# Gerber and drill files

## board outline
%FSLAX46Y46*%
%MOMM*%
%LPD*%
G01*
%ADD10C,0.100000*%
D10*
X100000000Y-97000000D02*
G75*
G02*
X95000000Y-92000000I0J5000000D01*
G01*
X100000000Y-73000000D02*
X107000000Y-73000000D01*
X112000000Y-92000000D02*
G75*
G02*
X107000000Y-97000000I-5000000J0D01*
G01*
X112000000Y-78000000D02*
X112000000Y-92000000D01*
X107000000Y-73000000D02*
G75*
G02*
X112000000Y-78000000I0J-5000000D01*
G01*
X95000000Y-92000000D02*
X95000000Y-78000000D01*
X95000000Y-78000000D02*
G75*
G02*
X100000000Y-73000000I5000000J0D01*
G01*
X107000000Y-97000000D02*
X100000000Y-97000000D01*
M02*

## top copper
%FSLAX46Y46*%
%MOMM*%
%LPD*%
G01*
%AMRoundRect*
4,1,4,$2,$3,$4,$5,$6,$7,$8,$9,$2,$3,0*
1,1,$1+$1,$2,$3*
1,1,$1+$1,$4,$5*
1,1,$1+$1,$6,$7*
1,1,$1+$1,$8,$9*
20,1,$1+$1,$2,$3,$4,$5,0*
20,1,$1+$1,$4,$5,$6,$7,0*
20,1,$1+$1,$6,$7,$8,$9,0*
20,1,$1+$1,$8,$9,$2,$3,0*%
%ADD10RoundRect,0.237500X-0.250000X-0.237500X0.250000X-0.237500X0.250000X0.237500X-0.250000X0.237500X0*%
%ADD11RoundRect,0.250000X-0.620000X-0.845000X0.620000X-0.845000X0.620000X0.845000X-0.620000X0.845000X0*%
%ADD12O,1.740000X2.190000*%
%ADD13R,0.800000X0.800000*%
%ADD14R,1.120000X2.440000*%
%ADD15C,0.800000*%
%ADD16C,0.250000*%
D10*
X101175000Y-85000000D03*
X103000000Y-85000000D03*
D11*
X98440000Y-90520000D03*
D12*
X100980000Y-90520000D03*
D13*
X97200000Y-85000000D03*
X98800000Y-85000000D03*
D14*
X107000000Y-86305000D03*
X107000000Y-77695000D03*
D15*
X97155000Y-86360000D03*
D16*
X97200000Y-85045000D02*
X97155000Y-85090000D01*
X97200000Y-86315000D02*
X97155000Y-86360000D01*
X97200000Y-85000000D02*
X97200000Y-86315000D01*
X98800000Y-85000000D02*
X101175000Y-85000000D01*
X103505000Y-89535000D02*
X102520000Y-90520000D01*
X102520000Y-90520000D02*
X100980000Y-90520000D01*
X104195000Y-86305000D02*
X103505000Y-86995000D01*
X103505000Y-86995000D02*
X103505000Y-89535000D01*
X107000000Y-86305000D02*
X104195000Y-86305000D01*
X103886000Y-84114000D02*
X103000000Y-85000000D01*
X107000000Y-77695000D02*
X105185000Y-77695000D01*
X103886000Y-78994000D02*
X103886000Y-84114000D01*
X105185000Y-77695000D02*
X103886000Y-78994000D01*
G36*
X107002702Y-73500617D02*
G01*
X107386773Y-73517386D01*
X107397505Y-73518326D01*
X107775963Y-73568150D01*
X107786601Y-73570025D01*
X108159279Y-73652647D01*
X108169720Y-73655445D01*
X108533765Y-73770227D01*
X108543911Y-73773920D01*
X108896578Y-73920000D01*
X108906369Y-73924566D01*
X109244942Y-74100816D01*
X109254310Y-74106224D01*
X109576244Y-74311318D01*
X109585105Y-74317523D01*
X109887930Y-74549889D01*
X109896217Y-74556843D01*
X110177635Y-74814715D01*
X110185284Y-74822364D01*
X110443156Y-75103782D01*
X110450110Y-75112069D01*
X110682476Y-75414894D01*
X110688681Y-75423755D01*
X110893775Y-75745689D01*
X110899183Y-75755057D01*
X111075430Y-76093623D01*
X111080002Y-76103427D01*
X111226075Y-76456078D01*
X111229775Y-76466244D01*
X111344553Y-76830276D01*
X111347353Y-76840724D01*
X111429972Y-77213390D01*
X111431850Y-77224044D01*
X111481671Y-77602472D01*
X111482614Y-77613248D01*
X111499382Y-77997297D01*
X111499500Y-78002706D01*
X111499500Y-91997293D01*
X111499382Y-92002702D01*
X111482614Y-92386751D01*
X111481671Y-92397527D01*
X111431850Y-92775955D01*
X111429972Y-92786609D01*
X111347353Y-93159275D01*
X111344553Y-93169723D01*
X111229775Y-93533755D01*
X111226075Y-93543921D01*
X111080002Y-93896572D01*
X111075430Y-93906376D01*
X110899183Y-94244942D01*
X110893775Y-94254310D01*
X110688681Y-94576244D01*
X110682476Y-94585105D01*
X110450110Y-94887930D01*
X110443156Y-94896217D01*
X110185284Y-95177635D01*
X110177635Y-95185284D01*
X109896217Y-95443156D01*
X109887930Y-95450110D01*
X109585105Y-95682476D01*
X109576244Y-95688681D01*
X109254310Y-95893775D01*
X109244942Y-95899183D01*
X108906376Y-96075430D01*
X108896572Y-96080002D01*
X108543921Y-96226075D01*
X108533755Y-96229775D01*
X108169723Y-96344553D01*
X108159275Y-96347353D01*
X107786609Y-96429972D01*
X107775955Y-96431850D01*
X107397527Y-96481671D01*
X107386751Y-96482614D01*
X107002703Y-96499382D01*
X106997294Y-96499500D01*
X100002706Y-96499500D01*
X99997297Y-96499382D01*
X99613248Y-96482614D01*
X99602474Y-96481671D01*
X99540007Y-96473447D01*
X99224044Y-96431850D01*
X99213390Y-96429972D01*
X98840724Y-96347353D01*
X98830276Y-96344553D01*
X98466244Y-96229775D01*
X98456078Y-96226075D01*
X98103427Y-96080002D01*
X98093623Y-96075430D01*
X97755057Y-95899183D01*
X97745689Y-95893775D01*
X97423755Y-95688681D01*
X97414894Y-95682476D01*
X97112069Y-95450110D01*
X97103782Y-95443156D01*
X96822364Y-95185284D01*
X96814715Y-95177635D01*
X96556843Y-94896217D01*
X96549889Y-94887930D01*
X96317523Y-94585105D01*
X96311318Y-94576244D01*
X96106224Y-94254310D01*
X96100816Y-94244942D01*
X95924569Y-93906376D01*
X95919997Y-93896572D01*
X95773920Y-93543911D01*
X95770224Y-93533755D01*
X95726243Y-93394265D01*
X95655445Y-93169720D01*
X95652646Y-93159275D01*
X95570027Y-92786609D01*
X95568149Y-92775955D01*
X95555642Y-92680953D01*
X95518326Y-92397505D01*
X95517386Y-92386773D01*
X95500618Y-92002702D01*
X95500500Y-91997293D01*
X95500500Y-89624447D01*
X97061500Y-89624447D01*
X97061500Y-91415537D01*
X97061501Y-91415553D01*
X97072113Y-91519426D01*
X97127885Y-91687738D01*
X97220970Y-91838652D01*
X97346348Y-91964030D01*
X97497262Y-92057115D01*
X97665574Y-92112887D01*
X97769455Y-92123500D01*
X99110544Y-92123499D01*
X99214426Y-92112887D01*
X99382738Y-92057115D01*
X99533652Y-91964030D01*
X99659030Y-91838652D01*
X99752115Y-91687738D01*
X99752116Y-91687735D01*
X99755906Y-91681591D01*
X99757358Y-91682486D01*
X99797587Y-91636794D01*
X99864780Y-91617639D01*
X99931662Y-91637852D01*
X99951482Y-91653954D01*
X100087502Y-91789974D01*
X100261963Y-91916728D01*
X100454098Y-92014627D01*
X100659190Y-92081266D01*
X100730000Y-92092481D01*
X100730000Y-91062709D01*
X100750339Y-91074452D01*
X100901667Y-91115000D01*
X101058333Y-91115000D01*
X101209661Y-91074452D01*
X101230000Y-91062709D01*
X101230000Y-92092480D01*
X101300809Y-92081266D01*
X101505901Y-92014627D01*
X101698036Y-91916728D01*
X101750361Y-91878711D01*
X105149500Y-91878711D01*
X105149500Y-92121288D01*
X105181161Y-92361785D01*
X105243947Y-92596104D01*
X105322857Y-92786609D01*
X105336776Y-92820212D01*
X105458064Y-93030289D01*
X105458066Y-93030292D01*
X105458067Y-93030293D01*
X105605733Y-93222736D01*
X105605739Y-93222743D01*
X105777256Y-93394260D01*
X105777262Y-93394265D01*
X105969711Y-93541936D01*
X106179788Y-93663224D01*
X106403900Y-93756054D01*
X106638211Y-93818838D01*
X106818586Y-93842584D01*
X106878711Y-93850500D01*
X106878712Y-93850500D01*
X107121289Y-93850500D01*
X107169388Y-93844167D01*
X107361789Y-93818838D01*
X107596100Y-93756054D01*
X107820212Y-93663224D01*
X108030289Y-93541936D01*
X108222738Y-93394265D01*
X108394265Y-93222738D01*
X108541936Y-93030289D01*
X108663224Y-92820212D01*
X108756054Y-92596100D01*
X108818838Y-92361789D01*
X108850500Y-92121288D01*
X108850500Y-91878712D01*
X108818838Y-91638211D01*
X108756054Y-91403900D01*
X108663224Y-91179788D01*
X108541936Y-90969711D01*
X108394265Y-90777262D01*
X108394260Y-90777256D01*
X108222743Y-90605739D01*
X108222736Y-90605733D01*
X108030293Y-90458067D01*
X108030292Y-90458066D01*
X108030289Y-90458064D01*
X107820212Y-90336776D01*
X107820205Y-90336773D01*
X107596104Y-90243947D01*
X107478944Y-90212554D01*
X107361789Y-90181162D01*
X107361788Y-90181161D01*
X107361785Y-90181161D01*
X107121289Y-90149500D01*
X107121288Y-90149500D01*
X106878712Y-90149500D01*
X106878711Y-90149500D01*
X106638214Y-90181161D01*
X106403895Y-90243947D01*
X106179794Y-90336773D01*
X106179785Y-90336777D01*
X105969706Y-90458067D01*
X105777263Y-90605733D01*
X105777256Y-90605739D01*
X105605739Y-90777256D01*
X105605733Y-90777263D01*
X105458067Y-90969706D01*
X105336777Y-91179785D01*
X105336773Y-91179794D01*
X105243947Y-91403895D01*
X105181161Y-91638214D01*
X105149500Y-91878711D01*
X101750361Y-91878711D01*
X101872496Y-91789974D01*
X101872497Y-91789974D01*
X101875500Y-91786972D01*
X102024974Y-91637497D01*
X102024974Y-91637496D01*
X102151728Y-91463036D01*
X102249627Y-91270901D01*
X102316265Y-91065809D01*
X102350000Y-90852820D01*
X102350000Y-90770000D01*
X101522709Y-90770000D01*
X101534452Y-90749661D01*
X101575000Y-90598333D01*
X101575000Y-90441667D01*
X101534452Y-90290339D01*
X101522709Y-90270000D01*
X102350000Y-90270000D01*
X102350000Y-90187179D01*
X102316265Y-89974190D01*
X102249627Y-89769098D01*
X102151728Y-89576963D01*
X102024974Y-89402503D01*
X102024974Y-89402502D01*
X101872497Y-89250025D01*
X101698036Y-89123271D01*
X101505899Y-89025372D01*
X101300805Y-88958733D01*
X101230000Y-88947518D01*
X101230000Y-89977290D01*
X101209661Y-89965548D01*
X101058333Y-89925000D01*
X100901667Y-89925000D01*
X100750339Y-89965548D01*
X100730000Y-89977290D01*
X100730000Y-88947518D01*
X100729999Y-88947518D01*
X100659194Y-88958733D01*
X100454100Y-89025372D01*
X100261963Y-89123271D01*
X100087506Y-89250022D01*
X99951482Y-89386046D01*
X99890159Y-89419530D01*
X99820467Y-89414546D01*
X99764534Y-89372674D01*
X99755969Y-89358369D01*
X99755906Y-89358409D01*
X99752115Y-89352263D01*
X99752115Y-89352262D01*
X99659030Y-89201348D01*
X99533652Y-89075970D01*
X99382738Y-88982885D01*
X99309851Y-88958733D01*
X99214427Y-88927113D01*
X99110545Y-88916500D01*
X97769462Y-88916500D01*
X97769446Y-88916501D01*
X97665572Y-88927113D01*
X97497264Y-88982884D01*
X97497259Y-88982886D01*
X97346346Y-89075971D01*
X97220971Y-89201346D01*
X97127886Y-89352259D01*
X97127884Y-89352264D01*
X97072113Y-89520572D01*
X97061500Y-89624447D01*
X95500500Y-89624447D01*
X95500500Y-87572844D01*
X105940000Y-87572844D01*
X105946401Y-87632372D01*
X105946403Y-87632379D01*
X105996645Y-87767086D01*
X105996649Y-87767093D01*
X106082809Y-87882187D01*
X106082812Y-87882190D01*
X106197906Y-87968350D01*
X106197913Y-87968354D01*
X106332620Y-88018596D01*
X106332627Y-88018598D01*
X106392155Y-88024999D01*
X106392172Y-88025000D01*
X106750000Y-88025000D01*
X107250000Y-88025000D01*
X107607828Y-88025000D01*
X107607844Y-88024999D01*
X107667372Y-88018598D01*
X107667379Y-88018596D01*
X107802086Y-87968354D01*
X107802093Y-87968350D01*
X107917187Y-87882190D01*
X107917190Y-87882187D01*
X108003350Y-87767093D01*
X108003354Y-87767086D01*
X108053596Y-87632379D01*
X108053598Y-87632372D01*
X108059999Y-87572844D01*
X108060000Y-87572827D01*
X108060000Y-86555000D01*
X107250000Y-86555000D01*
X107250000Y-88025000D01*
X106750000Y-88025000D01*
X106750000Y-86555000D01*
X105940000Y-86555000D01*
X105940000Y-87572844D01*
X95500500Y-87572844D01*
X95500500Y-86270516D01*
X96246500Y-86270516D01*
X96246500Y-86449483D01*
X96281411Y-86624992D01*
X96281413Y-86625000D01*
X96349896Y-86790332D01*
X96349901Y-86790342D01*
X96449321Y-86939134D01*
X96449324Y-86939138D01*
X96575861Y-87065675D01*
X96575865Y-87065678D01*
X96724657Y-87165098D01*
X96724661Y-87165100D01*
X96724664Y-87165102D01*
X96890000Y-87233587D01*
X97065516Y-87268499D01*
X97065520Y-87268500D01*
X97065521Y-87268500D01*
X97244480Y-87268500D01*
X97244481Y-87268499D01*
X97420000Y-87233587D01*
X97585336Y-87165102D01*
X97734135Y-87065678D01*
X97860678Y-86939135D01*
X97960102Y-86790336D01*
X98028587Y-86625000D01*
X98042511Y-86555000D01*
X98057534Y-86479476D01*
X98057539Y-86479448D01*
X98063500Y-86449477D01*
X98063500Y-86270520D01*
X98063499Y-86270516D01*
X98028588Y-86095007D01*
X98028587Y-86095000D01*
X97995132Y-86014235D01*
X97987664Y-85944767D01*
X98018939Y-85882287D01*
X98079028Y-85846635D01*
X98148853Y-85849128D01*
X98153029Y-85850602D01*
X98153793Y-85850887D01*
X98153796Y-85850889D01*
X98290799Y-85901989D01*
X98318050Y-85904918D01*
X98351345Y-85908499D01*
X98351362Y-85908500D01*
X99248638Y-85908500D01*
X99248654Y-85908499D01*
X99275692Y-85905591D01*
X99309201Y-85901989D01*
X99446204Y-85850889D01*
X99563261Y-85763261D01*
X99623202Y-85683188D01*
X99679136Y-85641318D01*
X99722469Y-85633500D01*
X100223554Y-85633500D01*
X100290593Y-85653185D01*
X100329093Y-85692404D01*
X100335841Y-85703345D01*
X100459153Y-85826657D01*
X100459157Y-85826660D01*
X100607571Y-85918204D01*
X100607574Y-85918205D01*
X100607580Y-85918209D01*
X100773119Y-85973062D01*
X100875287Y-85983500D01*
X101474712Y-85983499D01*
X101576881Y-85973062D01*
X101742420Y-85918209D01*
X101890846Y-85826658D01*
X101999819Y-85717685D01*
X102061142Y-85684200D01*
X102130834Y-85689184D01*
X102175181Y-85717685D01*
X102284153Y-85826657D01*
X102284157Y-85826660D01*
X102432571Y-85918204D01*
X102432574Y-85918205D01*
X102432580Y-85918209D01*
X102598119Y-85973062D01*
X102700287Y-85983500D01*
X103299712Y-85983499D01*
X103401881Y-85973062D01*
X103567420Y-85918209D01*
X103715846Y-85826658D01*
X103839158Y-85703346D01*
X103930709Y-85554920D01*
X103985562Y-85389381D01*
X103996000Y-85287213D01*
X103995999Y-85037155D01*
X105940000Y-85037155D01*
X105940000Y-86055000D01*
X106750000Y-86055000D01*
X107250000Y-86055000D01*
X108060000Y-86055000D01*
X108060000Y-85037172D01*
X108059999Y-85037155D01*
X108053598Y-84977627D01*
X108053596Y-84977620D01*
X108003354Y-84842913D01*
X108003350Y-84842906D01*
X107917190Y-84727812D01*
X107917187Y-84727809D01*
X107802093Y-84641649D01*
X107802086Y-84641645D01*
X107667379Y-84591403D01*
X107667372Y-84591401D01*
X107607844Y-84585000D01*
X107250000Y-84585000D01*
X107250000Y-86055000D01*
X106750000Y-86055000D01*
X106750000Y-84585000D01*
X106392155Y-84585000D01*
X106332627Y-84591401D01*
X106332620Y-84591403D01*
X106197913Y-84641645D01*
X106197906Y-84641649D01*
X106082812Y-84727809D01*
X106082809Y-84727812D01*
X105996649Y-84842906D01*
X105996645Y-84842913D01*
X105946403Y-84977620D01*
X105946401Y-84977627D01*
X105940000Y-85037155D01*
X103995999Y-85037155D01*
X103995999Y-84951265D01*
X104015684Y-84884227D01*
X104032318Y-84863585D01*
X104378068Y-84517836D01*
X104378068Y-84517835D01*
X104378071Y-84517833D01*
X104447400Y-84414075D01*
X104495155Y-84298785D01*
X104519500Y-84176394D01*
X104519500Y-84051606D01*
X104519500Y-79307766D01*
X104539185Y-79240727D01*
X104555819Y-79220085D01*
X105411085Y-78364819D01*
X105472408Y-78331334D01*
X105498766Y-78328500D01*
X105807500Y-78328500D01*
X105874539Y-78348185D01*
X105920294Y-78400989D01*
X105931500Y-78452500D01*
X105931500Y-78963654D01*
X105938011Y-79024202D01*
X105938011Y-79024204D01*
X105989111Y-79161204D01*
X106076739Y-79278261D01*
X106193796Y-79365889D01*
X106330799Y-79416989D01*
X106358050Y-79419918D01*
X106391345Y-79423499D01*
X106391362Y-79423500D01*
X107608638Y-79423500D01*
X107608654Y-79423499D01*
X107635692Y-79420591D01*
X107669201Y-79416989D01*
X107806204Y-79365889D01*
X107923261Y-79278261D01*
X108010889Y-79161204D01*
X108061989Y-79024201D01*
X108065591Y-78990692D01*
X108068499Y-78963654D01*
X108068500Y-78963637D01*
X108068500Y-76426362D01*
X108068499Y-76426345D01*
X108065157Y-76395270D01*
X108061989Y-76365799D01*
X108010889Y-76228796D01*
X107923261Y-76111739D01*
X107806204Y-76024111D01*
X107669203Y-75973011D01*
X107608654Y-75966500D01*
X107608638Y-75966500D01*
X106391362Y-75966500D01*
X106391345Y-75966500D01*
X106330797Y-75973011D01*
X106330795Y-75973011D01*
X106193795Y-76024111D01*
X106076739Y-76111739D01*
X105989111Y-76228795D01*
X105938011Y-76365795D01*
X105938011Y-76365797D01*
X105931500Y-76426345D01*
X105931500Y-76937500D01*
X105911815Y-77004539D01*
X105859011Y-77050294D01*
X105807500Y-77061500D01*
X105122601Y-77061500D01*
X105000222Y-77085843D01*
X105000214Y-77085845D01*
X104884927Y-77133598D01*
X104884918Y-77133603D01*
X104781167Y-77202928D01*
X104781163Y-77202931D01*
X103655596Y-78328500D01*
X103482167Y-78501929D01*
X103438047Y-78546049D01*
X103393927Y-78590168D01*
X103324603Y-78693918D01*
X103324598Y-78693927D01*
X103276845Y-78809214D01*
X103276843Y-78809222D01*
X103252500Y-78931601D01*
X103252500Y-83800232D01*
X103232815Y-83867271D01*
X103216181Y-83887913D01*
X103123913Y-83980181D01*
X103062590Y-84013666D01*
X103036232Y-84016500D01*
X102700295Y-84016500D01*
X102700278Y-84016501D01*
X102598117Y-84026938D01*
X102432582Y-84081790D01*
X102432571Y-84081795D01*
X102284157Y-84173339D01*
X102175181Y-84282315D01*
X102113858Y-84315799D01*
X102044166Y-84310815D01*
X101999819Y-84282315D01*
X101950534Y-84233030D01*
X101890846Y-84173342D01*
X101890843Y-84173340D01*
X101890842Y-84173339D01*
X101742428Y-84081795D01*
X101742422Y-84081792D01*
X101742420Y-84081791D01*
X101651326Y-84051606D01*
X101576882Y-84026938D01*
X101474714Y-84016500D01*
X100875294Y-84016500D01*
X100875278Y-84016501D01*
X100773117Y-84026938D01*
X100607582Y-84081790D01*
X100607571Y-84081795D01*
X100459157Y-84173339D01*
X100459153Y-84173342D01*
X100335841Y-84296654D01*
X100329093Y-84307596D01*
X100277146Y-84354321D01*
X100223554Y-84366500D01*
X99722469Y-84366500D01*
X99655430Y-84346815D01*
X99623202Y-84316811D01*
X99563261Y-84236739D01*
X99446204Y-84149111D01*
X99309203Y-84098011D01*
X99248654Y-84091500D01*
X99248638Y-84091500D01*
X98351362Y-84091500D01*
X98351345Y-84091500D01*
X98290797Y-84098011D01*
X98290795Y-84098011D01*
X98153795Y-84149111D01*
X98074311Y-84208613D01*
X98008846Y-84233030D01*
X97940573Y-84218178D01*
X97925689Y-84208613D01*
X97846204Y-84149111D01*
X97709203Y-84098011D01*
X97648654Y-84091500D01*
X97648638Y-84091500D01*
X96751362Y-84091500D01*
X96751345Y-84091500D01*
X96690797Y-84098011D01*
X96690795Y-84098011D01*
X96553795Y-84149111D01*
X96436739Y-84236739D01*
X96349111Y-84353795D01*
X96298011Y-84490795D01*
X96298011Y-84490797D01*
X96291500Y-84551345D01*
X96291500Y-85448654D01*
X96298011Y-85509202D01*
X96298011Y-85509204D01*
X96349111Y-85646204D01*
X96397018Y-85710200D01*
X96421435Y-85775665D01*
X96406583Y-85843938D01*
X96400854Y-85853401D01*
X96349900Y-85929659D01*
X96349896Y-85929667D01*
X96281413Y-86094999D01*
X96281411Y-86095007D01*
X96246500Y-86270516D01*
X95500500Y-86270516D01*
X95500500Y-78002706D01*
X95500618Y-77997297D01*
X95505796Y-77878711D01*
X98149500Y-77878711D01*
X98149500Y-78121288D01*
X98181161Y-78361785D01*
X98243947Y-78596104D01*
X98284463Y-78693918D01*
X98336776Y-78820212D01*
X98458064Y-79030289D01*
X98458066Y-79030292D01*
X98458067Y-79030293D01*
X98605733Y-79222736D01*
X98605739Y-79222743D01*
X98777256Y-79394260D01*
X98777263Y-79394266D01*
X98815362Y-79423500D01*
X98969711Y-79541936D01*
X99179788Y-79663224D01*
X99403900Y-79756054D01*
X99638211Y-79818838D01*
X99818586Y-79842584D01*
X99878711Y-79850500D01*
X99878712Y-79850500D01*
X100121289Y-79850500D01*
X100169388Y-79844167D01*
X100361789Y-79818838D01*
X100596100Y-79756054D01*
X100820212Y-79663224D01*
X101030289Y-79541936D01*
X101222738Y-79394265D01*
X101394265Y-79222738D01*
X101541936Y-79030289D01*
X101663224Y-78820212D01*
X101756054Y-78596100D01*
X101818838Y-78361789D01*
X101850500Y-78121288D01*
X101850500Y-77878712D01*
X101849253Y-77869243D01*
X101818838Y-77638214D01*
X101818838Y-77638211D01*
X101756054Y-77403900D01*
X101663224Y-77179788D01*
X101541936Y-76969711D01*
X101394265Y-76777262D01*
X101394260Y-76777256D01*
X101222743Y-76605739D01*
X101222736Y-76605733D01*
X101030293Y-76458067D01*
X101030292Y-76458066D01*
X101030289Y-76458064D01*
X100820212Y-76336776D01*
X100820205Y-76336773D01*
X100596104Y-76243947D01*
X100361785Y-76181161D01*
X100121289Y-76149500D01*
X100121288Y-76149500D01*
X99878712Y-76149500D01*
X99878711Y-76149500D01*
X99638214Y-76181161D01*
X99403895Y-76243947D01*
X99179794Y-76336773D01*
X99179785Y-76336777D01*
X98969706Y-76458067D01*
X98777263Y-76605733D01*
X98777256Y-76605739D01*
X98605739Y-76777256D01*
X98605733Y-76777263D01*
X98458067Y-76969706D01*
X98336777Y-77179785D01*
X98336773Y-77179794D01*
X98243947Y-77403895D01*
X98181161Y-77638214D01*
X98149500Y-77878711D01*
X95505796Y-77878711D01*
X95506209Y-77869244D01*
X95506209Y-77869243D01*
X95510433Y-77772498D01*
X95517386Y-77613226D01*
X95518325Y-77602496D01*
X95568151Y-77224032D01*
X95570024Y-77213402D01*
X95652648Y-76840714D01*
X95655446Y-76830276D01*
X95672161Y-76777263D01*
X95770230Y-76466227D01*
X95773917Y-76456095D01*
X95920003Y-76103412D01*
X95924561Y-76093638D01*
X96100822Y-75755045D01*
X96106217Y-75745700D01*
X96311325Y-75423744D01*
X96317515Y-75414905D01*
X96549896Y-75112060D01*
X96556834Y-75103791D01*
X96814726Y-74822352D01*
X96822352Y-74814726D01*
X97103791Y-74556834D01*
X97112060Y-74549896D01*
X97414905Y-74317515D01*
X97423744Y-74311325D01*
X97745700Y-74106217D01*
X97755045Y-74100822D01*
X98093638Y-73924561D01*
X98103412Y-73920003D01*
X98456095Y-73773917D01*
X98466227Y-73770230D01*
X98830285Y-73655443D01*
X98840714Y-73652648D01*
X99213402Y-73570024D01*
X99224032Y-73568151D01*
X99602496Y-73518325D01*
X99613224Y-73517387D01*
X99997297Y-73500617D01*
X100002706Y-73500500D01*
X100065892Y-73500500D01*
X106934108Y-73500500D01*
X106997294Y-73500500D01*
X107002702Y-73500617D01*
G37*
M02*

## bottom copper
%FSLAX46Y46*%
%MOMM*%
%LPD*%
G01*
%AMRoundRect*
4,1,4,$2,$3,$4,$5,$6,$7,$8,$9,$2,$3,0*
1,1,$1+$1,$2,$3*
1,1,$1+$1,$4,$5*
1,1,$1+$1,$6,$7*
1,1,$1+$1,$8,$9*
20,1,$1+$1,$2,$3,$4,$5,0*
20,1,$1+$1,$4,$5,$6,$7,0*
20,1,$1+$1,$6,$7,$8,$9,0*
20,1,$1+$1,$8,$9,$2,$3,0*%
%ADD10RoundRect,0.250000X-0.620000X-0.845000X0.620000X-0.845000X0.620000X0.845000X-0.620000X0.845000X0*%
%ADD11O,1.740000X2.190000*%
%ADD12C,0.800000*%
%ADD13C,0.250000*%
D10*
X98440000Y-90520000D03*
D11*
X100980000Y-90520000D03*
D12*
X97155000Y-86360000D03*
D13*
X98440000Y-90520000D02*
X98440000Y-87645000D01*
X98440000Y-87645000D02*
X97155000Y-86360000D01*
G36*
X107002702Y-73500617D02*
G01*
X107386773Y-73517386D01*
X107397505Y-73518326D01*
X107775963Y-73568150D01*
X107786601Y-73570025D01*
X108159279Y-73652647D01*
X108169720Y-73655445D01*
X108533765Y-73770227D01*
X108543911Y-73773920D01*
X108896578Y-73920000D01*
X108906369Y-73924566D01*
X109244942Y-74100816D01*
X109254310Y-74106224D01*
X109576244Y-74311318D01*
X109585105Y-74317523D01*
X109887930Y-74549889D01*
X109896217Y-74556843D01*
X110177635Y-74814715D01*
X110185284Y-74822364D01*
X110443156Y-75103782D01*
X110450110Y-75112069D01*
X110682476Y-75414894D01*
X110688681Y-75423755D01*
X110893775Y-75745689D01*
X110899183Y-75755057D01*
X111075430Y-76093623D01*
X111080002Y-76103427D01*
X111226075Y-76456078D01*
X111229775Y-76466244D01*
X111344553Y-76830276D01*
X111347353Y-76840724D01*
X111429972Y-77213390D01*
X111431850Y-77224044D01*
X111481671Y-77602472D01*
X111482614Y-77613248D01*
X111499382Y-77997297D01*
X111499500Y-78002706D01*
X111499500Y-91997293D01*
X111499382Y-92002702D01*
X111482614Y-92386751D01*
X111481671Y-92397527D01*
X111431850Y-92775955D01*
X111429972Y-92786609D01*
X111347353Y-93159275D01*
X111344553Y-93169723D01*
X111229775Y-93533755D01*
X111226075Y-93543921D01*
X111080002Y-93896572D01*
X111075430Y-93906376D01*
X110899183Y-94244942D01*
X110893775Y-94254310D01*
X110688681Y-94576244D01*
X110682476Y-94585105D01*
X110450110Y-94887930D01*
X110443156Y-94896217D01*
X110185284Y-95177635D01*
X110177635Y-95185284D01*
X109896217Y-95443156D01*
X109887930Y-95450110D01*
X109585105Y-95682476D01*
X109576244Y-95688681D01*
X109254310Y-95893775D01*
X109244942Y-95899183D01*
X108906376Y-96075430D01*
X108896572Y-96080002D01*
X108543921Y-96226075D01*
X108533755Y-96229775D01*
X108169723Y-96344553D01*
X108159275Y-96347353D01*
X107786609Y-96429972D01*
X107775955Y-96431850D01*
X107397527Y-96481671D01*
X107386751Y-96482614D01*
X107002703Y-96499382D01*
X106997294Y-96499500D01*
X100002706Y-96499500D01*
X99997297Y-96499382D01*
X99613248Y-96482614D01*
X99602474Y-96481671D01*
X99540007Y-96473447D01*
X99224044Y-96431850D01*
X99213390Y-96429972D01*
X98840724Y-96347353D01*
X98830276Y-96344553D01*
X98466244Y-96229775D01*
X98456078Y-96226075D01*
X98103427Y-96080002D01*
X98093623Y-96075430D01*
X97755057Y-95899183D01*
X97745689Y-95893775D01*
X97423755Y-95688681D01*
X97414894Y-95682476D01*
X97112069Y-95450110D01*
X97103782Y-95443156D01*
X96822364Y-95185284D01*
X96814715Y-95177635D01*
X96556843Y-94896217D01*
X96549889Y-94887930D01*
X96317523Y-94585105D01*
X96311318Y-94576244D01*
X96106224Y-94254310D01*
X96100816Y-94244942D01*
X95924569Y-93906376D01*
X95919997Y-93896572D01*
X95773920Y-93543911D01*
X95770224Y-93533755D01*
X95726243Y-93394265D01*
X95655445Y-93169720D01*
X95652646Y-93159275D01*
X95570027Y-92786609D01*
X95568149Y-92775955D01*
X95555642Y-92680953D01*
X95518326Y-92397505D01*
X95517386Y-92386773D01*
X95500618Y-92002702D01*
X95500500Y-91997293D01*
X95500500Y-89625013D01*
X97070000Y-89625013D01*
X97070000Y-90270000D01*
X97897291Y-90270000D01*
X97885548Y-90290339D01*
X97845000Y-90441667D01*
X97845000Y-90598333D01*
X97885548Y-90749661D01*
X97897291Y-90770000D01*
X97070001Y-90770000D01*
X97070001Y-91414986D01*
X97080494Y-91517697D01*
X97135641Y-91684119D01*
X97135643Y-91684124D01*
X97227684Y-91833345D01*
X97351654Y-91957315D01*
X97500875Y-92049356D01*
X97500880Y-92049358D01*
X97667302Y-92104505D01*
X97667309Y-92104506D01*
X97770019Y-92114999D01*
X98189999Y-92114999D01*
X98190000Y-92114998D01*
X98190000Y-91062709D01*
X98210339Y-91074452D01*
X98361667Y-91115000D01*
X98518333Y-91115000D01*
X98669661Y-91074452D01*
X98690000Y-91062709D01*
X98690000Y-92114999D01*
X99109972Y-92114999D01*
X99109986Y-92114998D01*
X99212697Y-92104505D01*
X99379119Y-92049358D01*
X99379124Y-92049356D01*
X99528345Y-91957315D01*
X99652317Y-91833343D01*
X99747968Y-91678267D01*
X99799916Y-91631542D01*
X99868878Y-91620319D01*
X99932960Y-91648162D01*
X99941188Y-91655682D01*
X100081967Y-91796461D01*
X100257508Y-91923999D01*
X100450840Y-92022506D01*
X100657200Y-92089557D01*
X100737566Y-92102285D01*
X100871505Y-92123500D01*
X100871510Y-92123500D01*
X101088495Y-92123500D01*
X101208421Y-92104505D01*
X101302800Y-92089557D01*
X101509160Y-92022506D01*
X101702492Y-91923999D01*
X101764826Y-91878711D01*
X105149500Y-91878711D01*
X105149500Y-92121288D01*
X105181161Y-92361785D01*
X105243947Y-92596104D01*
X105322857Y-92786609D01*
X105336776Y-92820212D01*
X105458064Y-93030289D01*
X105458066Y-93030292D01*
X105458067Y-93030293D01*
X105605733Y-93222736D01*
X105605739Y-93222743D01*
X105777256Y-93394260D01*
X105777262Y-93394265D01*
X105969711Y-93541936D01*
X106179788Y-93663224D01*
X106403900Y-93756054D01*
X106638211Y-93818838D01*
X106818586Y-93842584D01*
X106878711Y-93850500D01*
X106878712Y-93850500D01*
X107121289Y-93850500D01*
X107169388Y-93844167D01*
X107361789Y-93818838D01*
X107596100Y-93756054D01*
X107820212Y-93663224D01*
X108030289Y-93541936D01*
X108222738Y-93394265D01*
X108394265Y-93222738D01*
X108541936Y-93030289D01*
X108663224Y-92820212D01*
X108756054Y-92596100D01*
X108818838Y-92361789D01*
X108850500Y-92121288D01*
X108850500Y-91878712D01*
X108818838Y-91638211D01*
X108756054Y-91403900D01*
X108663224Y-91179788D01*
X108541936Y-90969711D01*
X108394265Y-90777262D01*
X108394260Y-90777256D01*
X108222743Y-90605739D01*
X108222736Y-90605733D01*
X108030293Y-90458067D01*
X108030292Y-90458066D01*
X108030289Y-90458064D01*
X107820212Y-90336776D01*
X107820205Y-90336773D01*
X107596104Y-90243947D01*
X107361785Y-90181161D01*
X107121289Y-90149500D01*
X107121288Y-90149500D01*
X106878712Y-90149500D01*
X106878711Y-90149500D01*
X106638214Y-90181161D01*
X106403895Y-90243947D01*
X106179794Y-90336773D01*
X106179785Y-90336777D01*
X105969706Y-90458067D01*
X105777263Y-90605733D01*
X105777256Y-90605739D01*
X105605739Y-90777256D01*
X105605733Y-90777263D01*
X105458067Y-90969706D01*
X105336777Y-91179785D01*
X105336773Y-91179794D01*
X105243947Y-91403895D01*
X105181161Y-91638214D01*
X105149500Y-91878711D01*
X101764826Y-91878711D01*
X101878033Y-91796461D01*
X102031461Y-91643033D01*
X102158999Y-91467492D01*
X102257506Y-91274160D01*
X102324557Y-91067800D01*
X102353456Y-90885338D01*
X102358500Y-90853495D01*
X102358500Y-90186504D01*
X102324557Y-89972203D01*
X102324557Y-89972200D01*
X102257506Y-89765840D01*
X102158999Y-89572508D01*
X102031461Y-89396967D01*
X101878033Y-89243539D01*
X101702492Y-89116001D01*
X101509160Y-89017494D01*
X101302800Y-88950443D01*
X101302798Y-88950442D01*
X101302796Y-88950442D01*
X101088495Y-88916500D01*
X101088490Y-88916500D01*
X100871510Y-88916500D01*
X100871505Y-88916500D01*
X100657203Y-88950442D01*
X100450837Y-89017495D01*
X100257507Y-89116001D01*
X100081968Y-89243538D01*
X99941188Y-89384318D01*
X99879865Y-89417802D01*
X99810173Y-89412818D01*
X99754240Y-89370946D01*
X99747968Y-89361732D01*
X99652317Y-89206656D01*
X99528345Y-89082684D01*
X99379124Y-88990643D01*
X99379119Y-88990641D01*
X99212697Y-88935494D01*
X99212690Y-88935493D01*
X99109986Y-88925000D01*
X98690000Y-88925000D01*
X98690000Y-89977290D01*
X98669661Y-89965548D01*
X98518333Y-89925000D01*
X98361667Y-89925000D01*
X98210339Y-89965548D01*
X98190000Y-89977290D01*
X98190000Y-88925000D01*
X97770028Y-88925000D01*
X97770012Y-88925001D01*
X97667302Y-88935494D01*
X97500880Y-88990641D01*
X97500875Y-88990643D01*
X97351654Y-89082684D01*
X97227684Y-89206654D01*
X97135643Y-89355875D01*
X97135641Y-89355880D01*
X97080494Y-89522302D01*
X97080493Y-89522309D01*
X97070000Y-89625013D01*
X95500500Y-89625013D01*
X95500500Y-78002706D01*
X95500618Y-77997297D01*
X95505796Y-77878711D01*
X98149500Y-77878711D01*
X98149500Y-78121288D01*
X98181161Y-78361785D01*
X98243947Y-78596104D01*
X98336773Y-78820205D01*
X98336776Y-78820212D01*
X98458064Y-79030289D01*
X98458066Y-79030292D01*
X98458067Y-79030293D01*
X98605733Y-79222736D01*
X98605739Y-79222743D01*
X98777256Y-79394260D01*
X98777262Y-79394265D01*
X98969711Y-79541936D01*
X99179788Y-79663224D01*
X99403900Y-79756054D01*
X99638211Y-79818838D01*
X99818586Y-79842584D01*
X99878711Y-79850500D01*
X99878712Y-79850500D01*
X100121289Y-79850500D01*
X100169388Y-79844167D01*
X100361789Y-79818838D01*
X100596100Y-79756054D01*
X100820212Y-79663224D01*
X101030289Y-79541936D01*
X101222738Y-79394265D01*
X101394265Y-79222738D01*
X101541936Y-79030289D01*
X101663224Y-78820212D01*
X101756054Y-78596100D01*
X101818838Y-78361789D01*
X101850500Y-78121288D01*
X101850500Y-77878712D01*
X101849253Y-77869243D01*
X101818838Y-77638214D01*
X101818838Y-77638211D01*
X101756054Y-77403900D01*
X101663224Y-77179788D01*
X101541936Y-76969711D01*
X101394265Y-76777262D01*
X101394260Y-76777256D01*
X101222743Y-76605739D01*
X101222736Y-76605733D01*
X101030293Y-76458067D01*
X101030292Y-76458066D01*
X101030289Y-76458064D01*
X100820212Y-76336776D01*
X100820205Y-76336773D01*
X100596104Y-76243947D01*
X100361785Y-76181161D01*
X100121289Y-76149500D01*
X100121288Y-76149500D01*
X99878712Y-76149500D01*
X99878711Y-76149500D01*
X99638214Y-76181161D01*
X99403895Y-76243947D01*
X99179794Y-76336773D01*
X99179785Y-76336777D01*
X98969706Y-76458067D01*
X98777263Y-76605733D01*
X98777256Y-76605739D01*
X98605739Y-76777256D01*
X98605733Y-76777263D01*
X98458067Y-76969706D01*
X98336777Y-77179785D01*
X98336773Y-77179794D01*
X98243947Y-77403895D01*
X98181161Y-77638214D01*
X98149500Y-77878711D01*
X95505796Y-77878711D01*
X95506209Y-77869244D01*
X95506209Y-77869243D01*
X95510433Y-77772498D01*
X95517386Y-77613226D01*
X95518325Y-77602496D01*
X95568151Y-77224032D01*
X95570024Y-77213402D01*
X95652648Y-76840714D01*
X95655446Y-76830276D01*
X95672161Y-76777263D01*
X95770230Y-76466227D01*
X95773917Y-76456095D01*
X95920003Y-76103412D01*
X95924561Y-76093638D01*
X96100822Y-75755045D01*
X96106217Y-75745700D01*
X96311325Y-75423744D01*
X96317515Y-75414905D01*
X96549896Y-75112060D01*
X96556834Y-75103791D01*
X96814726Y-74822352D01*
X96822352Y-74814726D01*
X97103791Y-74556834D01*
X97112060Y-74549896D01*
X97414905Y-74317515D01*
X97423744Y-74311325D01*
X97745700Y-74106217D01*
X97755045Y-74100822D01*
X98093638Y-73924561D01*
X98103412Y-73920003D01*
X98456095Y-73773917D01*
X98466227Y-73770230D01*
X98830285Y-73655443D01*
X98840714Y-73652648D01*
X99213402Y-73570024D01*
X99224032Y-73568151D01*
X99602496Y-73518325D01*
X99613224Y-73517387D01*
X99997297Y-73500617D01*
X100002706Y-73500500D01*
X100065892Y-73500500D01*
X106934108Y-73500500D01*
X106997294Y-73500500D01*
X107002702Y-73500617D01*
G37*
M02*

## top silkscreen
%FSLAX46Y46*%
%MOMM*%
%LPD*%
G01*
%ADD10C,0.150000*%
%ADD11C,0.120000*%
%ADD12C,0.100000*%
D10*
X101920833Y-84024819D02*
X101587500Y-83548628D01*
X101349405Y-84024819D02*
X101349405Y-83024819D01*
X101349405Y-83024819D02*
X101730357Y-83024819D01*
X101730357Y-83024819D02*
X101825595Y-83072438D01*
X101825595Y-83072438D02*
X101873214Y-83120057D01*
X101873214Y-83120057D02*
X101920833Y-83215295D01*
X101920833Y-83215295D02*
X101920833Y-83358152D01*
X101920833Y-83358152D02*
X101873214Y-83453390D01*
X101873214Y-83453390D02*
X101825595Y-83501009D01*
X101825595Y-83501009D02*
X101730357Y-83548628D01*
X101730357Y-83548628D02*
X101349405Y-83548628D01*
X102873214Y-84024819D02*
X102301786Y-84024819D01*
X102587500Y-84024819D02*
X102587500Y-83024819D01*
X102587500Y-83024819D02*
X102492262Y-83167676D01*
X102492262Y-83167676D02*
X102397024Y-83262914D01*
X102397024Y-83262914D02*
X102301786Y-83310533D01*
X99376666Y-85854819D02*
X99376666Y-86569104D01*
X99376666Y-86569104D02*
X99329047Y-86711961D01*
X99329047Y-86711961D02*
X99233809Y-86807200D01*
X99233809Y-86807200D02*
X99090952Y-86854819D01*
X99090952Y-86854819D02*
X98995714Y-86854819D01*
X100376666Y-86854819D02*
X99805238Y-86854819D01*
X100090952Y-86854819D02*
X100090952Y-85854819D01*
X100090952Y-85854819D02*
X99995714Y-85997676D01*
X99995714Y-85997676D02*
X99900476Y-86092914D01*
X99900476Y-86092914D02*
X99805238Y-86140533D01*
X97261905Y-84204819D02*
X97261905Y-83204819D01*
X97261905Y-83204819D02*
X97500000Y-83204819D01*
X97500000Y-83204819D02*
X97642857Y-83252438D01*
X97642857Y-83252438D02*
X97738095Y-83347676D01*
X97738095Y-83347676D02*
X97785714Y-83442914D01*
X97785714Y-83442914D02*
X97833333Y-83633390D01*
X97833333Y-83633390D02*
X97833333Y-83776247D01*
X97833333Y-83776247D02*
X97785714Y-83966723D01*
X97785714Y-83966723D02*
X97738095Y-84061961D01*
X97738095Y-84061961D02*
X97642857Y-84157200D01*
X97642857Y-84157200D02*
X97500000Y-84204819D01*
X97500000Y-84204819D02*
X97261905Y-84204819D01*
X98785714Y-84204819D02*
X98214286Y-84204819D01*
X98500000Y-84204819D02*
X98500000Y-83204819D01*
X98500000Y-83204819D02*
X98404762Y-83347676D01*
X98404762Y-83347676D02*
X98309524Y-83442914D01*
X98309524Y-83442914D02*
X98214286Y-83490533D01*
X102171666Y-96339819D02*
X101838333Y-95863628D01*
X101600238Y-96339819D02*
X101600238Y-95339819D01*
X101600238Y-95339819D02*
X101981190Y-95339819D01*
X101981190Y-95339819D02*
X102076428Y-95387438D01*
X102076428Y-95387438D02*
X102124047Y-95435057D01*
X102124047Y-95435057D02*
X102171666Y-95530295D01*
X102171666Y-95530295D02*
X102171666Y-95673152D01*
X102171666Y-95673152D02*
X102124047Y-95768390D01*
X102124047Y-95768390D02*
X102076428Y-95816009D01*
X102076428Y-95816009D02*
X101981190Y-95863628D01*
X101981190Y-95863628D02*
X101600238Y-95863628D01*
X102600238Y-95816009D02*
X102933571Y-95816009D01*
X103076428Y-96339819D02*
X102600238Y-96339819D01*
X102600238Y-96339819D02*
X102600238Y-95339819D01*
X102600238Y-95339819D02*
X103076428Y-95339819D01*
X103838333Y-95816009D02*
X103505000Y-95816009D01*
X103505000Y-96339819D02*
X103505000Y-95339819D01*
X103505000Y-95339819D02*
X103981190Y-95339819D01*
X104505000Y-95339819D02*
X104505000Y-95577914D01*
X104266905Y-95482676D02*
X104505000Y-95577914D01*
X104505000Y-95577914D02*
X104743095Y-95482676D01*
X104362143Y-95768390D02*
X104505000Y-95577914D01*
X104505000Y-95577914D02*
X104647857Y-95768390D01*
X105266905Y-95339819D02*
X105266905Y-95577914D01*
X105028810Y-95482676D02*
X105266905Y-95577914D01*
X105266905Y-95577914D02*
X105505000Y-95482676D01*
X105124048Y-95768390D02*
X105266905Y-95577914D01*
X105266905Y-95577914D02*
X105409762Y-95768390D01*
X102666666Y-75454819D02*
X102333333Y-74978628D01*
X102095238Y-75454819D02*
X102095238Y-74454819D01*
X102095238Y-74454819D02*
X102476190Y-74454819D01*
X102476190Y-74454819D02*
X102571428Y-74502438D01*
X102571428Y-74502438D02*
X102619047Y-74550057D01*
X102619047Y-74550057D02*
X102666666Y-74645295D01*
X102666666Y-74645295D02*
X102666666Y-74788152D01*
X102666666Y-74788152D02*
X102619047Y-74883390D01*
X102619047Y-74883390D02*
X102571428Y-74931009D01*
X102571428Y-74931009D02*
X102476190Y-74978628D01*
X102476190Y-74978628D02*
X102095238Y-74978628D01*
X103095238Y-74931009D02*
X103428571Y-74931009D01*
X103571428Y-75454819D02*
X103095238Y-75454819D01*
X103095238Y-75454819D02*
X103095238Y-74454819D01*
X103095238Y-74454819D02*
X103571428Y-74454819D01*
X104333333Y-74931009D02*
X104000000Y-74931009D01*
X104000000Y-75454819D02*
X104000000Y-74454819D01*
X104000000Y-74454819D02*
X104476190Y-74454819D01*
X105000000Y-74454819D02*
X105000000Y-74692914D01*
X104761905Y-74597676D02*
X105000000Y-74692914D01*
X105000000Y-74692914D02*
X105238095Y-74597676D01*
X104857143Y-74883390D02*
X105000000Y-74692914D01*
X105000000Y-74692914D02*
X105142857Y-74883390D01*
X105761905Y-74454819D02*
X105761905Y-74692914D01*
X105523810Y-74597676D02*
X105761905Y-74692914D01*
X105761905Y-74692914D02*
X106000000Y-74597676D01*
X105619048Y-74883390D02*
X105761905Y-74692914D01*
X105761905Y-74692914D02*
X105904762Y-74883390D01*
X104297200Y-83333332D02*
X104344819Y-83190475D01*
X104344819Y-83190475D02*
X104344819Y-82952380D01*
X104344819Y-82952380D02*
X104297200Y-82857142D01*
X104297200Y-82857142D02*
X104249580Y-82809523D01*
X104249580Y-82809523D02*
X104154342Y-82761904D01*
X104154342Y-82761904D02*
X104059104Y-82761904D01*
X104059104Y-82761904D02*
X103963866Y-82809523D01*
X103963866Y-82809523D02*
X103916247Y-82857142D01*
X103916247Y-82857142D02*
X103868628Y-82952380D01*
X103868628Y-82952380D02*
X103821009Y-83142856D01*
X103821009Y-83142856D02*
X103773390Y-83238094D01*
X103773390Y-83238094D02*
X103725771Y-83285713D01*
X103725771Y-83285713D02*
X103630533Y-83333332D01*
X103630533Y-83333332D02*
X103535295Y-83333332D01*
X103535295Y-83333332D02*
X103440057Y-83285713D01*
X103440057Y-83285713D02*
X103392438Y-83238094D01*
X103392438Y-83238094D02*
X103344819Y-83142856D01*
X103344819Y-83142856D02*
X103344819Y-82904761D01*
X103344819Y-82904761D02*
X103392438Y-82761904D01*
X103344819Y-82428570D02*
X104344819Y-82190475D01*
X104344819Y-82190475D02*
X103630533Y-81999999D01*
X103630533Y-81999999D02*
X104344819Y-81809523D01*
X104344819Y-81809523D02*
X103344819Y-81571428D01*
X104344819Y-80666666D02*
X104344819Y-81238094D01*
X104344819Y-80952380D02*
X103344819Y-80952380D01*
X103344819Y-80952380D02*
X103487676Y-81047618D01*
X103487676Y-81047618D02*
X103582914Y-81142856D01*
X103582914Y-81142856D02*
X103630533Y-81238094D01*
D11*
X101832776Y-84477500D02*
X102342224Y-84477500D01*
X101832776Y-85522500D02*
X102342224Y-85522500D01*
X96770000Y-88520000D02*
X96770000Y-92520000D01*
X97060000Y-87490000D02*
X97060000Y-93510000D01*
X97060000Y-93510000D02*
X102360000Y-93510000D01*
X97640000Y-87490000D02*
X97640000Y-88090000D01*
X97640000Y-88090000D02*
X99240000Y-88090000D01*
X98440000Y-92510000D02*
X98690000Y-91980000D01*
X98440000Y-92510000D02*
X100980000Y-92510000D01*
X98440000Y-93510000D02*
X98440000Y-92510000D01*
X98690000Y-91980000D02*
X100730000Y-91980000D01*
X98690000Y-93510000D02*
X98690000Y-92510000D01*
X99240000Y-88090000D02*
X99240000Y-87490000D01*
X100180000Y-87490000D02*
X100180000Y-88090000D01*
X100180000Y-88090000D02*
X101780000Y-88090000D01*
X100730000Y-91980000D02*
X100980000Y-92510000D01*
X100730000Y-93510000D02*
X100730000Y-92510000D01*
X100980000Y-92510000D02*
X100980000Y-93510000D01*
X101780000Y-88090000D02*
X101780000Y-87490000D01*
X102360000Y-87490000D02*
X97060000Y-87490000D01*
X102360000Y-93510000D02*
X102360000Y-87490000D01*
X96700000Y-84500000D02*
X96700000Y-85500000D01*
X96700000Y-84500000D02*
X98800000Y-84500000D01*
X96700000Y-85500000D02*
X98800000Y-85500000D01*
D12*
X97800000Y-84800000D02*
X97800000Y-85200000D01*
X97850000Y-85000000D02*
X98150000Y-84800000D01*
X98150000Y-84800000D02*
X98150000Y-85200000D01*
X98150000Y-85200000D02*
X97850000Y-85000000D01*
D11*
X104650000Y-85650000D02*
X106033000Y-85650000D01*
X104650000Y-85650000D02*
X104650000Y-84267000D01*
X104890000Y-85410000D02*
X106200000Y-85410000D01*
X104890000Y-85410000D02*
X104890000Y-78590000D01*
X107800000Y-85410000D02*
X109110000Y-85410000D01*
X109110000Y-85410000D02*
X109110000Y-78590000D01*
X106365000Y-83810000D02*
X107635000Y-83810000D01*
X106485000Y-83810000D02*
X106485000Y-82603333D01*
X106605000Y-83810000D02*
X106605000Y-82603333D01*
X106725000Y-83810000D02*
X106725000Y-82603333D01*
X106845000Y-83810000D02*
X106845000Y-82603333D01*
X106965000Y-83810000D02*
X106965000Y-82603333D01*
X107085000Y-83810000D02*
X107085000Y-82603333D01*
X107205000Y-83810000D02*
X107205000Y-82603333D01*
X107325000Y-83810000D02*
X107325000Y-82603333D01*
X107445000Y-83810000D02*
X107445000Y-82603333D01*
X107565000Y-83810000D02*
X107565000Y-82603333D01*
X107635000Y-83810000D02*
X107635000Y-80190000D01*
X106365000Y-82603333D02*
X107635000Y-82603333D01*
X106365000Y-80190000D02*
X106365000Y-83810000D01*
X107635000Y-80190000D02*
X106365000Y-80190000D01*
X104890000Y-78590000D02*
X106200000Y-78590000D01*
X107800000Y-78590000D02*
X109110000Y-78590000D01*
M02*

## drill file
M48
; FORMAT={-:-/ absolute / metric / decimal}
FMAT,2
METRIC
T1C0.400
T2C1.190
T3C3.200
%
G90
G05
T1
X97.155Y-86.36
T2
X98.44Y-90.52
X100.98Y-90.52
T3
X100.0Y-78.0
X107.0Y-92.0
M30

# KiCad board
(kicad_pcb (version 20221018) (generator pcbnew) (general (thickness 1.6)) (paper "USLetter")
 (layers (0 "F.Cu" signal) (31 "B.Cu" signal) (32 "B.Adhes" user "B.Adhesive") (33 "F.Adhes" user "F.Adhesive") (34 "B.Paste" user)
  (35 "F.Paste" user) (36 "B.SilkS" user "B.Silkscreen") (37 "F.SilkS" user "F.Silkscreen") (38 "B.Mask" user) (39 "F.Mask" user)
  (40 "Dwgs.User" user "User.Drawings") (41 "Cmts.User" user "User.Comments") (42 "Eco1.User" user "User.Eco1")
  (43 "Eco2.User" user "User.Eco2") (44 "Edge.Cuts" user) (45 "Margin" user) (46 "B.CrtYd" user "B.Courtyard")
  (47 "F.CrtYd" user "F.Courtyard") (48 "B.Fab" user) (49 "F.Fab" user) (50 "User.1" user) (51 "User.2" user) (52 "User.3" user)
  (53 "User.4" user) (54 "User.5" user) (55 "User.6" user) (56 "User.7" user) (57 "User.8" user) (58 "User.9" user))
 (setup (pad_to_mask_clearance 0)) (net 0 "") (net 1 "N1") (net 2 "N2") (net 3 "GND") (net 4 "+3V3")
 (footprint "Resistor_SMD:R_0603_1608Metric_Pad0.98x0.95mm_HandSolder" (layer "F.Cu") (at 102.0875 85)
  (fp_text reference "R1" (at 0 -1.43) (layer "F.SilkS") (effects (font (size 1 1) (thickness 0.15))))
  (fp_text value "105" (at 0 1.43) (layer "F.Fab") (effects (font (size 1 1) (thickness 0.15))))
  (fp_line (start -0.254724 -0.5225) (end 0.254724 -0.5225) (stroke (width 0.12) (type solid)) (layer "F.SilkS"))
  (fp_line (start -0.254724 0.5225) (end 0.254724 0.5225) (stroke (width 0.12) (type solid)) (layer "F.SilkS"))
  (pad "1" smd roundrect (at -0.9125 0) (size 0.975 0.95) (layers "F.Cu" "F.Paste" "F.Mask") (roundrect_rratio 0.25) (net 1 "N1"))
  (pad "2" smd roundrect (at 0.9125 0) (size 0.975 0.95) (layers "F.Cu" "F.Paste" "F.Mask") (roundrect_rratio 0.25) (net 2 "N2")))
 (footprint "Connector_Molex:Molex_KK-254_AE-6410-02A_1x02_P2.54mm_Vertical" (layer "F.Cu") (at 98.44 90.52)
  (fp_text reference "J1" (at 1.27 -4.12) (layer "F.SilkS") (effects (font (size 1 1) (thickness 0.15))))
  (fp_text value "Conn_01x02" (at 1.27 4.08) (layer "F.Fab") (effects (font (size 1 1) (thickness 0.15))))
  (fp_line (start -1.67 -2) (end -1.67 2) (stroke (width 0.12) (type solid)) (layer "F.SilkS"))
  (fp_line (start -1.38 -3.03) (end -1.38 2.99) (stroke (width 0.12) (type solid)) (layer "F.SilkS"))
  (fp_line (start -1.38 2.99) (end 3.92 2.99) (stroke (width 0.12) (type solid)) (layer "F.SilkS"))
  (fp_line (start -0.8 -3.03) (end -0.8 -2.43) (stroke (width 0.12) (type solid)) (layer "F.SilkS"))
  (fp_line (start -0.8 -2.43) (end 0.8 -2.43) (stroke (width 0.12) (type solid)) (layer "F.SilkS"))
  (fp_line (start 0 1.99) (end 0.25 1.46) (stroke (width 0.12) (type solid)) (layer "F.SilkS"))
  (fp_line (start 0 1.99) (end 2.54 1.99) (stroke (width 0.12) (type solid)) (layer "F.SilkS"))
  (fp_line (start 0 2.99) (end 0 1.99) (stroke (width 0.12) (type solid)) (layer "F.SilkS"))
  (fp_line (start 0.25 1.46) (end 2.29 1.46) (stroke (width 0.12) (type solid)) (layer "F.SilkS"))
  (fp_line (start 0.25 2.99) (end 0.25 1.99) (stroke (width 0.12) (type solid)) (layer "F.SilkS"))
  (fp_line (start 0.8 -2.43) (end 0.8 -3.03) (stroke (width 0.12) (type solid)) (layer "F.SilkS"))
  (fp_line (start 1.74 -3.03) (end 1.74 -2.43) (stroke (width 0.12) (type solid)) (layer "F.SilkS"))
  (fp_line (start 1.74 -2.43) (end 3.34 -2.43) (stroke (width 0.12) (type solid)) (layer "F.SilkS"))
  (fp_line (start 2.29 1.46) (end 2.54 1.99) (stroke (width 0.12) (type solid)) (layer "F.SilkS"))
  (fp_line (start 2.29 2.99) (end 2.29 1.99) (stroke (width 0.12) (type solid)) (layer "F.SilkS"))
  (fp_line (start 2.54 1.99) (end 2.54 2.99) (stroke (width 0.12) (type solid)) (layer "F.SilkS"))
  (fp_line (start 3.34 -2.43) (end 3.34 -3.03) (stroke (width 0.12) (type solid)) (layer "F.SilkS"))
  (fp_line (start 3.92 -3.03) (end -1.38 -3.03) (stroke (width 0.12) (type solid)) (layer "F.SilkS"))
  (fp_line (start 3.92 2.99) (end 3.92 -3.03) (stroke (width 0.12) (type solid)) (layer "F.SilkS"))
  (pad "1" thru_hole roundrect (at 0 0) (size 1.74 2.19) (drill 1.19) (layers "*.Cu" "*.Mask") (roundrect_rratio 0.143678) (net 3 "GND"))
  (pad "2" thru_hole oval (at 2.54 0) (size 1.74 2.19) (drill 1.19) (layers "*.Cu" "*.Mask") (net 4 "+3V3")))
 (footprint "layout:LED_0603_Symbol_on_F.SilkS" (layer "F.Cu") (at 98 85)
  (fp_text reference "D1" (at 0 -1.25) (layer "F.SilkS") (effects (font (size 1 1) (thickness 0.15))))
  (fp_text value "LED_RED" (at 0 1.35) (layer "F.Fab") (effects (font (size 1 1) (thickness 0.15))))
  (fp_line (start -1.3 -0.5) (end -1.3 0.5) (stroke (width 0.12) (type solid)) (layer "F.SilkS"))
  (fp_line (start -1.3 -0.5) (end 0.8 -0.5) (stroke (width 0.12) (type solid)) (layer "F.SilkS"))
  (fp_line (start -1.3 0.5) (end 0.8 0.5) (stroke (width 0.12) (type solid)) (layer "F.SilkS"))
  (fp_line (start -0.2 -0.2) (end -0.2 0.2) (stroke (width 0.1) (type solid)) (layer "F.SilkS"))
  (fp_line (start -0.15 0) (end 0.15 -0.2) (stroke (width 0.1) (type solid)) (layer "F.SilkS"))
  (fp_line (start 0.15 -0.2) (end 0.15 0.2) (stroke (width 0.1) (type solid)) (layer "F.SilkS"))
  (fp_line (start 0.15 0.2) (end -0.15 0) (stroke (width 0.1) (type solid)) (layer "F.SilkS"))
  (pad "1" smd rect (at -0.8 0 180) (size 0.8 0.8) (layers "F.Cu" "F.Paste" "F.Mask") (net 3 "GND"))
  (pad "2" smd rect (at 0.8 0 180) (size 0.8 0.8) (layers "F.Cu" "F.Paste" "F.Mask") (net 1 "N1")))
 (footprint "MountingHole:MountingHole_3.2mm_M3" (layer "F.Cu") (at 107 92)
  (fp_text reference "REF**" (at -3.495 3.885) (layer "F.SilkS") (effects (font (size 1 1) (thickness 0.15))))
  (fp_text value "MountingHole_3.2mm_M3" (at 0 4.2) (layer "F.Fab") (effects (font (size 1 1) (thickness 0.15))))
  (pad "" np_thru_hole circle (at 0 0) (size 3.2 3.2) (drill 3.2) (layers "F&B.Cu" "*.Mask")))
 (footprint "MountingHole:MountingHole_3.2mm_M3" (layer "F.Cu") (at 100 78)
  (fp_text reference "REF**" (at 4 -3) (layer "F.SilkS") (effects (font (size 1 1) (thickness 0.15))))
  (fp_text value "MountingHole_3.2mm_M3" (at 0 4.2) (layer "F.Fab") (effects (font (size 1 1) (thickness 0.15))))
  (pad "" np_thru_hole circle (at 0 0) (size 3.2 3.2) (drill 3.2) (layers "*.Cu" "*.Mask")))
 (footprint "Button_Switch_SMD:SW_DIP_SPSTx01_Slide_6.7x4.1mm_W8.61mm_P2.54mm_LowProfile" (layer "F.Cu") (at 107 82 90)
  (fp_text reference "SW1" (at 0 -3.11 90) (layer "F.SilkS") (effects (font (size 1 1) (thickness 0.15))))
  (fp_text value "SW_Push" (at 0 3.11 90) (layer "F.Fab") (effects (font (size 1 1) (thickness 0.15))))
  (fp_line (start -3.65 -2.35) (end -3.65 -0.967) (stroke (width 0.12) (type solid)) (layer "F.SilkS"))
  (fp_line (start -3.65 -2.35) (end -2.267 -2.35) (stroke (width 0.12) (type solid)) (layer "F.SilkS"))
  (fp_line (start -3.41 -2.11) (end -3.41 -0.8) (stroke (width 0.12) (type solid)) (layer "F.SilkS"))
  (fp_line (start -3.41 -2.11) (end 3.41 -2.11) (stroke (width 0.12) (type solid)) (layer "F.SilkS"))
  (fp_line (start -3.41 0.8) (end -3.41 2.11) (stroke (width 0.12) (type solid)) (layer "F.SilkS"))
  (fp_line (start -3.41 2.11) (end 3.41 2.11) (stroke (width 0.12) (type solid)) (layer "F.SilkS"))
  (fp_line (start -1.81 -0.635) (end -1.81 0.635) (stroke (width 0.12) (type solid)) (layer "F.SilkS"))
  (fp_line (start -1.81 -0.515) (end -0.603333 -0.515) (stroke (width 0.12) (type solid)) (layer "F.SilkS"))
  (fp_line (start -1.81 -0.395) (end -0.603333 -0.395) (stroke (width 0.12) (type solid)) (layer "F.SilkS"))
  (fp_line (start -1.81 -0.275) (end -0.603333 -0.275) (stroke (width 0.12) (type solid)) (layer "F.SilkS"))
  (fp_line (start -1.81 -0.155) (end -0.603333 -0.155) (stroke (width 0.12) (type solid)) (layer "F.SilkS"))
  (fp_line (start -1.81 -0.035) (end -0.603333 -0.035) (stroke (width 0.12) (type solid)) (layer "F.SilkS"))
  (fp_line (start -1.81 0.085) (end -0.603333 0.085) (stroke (width 0.12) (type solid)) (layer "F.SilkS"))
  (fp_line (start -1.81 0.205) (end -0.603333 0.205) (stroke (width 0.12) (type solid)) (layer "F.SilkS"))
  (fp_line (start -1.81 0.325) (end -0.603333 0.325) (stroke (width 0.12) (type solid)) (layer "F.SilkS"))
  (fp_line (start -1.81 0.445) (end -0.603333 0.445) (stroke (width 0.12) (type solid)) (layer "F.SilkS"))
  (fp_line (start -1.81 0.565) (end -0.603333 0.565) (stroke (width 0.12) (type solid)) (layer "F.SilkS"))
  (fp_line (start -1.81 0.635) (end 1.81 0.635) (stroke (width 0.12) (type solid)) (layer "F.SilkS"))
  (fp_line (start -0.603333 -0.635) (end -0.603333 0.635) (stroke (width 0.12) (type solid)) (layer "F.SilkS"))
  (fp_line (start 1.81 -0.635) (end -1.81 -0.635) (stroke (width 0.12) (type solid)) (layer "F.SilkS"))
  (fp_line (start 1.81 0.635) (end 1.81 -0.635) (stroke (width 0.12) (type solid)) (layer "F.SilkS"))
  (fp_line (start 3.41 -2.11) (end 3.41 -0.8) (stroke (width 0.12) (type solid)) (layer "F.SilkS"))
  (fp_line (start 3.41 0.8) (end 3.41 2.11) (stroke (width 0.12) (type solid)) (layer "F.SilkS"))
  (pad "1" smd rect (at -4.305 0 90) (size 2.44 1.12) (layers "F.Cu" "F.Paste" "F.Mask") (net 4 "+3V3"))
  (pad "2" smd rect (at 4.305 0 90) (size 2.44 1.12) (layers "F.Cu" "F.Paste" "F.Mask") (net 2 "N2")))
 (gr_arc (start 100 97) (mid 96.464466 95.535534) (end 95 92) (stroke (width 0.1) (type default)) (layer "Edge.Cuts"))
 (gr_line (start 100 73) (end 107 73) (stroke (width 0.1) (type default)) (layer "Edge.Cuts"))
 (gr_arc (start 112 92) (mid 110.535534 95.535534) (end 107 97) (stroke (width 0.1) (type default)) (layer "Edge.Cuts"))
 (gr_line (start 112 78) (end 112 92) (stroke (width 0.1) (type default)) (layer "Edge.Cuts"))
 (gr_arc (start 107 73) (mid 110.535534 74.464466) (end 112 78) (stroke (width 0.1) (type default)) (layer "Edge.Cuts"))
 (gr_line (start 95 92) (end 95 78) (stroke (width 0.1) (type default)) (layer "Edge.Cuts"))
 (gr_arc (start 95 78) (mid 96.464466 74.464466) (end 100 73) (stroke (width 0.1) (type default)) (layer "Edge.Cuts"))
 (gr_line (start 107 97) (end 100 97) (stroke (width 0.1) (type default)) (layer "Edge.Cuts"))
 (segment (start 97.2 85.045) (end 97.155 85.09) (width 0.25) (layer "F.Cu") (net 3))
 (segment (start 97.2 86.315) (end 97.155 86.36) (width 0.25) (layer "F.Cu") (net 3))
 (segment (start 97.2 85) (end 97.2 86.315) (width 0.25) (layer "F.Cu") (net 3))
 (via (at 97.155 86.36) (size 0.8) (drill 0.4) (layers "F.Cu" "B.Cu") (free) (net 3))
 (segment (start 98.44 90.52) (end 98.44 87.645) (width 0.25) (layer "B.Cu") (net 3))
 (segment (start 98.44 87.645) (end 97.155 86.36) (width 0.25) (layer "B.Cu") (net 3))
 (segment (start 98.8 85) (end 101.175 85) (width 0.25) (layer "F.Cu") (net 1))
 (segment (start 103.505 89.535) (end 102.52 90.52) (width 0.25) (layer "F.Cu") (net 4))
 (segment (start 102.52 90.52) (end 100.98 90.52) (width 0.25) (layer "F.Cu") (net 4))
 (segment (start 104.195 86.305) (end 103.505 86.995) (width 0.25) (layer "F.Cu") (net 4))
 (segment (start 103.505 86.995) (end 103.505 89.535) (width 0.25) (layer "F.Cu") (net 4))
 (segment (start 107 86.305) (end 104.195 86.305) (width 0.25) (layer "F.Cu") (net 4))
 (segment (start 103.886 84.114) (end 103 85) (width 0.25) (layer "F.Cu") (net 2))
 (segment (start 107 77.695) (end 105.185 77.695) (width 0.25) (layer "F.Cu") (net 2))
 (segment (start 103.886 78.994) (end 103.886 84.114) (width 0.25) (layer "F.Cu") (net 2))
 (segment (start 105.185 77.695) (end 103.886 78.994) (width 0.25) (layer "F.Cu") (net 2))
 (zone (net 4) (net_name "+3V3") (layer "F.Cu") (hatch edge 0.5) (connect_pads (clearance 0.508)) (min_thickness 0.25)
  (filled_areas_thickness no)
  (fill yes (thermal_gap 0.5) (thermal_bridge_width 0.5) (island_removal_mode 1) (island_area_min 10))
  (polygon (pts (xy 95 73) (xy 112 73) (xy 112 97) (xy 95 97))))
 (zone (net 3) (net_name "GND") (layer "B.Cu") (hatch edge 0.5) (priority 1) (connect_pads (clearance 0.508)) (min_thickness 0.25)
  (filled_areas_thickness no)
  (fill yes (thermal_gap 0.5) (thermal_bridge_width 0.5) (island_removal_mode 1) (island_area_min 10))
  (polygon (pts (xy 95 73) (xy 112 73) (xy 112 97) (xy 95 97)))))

